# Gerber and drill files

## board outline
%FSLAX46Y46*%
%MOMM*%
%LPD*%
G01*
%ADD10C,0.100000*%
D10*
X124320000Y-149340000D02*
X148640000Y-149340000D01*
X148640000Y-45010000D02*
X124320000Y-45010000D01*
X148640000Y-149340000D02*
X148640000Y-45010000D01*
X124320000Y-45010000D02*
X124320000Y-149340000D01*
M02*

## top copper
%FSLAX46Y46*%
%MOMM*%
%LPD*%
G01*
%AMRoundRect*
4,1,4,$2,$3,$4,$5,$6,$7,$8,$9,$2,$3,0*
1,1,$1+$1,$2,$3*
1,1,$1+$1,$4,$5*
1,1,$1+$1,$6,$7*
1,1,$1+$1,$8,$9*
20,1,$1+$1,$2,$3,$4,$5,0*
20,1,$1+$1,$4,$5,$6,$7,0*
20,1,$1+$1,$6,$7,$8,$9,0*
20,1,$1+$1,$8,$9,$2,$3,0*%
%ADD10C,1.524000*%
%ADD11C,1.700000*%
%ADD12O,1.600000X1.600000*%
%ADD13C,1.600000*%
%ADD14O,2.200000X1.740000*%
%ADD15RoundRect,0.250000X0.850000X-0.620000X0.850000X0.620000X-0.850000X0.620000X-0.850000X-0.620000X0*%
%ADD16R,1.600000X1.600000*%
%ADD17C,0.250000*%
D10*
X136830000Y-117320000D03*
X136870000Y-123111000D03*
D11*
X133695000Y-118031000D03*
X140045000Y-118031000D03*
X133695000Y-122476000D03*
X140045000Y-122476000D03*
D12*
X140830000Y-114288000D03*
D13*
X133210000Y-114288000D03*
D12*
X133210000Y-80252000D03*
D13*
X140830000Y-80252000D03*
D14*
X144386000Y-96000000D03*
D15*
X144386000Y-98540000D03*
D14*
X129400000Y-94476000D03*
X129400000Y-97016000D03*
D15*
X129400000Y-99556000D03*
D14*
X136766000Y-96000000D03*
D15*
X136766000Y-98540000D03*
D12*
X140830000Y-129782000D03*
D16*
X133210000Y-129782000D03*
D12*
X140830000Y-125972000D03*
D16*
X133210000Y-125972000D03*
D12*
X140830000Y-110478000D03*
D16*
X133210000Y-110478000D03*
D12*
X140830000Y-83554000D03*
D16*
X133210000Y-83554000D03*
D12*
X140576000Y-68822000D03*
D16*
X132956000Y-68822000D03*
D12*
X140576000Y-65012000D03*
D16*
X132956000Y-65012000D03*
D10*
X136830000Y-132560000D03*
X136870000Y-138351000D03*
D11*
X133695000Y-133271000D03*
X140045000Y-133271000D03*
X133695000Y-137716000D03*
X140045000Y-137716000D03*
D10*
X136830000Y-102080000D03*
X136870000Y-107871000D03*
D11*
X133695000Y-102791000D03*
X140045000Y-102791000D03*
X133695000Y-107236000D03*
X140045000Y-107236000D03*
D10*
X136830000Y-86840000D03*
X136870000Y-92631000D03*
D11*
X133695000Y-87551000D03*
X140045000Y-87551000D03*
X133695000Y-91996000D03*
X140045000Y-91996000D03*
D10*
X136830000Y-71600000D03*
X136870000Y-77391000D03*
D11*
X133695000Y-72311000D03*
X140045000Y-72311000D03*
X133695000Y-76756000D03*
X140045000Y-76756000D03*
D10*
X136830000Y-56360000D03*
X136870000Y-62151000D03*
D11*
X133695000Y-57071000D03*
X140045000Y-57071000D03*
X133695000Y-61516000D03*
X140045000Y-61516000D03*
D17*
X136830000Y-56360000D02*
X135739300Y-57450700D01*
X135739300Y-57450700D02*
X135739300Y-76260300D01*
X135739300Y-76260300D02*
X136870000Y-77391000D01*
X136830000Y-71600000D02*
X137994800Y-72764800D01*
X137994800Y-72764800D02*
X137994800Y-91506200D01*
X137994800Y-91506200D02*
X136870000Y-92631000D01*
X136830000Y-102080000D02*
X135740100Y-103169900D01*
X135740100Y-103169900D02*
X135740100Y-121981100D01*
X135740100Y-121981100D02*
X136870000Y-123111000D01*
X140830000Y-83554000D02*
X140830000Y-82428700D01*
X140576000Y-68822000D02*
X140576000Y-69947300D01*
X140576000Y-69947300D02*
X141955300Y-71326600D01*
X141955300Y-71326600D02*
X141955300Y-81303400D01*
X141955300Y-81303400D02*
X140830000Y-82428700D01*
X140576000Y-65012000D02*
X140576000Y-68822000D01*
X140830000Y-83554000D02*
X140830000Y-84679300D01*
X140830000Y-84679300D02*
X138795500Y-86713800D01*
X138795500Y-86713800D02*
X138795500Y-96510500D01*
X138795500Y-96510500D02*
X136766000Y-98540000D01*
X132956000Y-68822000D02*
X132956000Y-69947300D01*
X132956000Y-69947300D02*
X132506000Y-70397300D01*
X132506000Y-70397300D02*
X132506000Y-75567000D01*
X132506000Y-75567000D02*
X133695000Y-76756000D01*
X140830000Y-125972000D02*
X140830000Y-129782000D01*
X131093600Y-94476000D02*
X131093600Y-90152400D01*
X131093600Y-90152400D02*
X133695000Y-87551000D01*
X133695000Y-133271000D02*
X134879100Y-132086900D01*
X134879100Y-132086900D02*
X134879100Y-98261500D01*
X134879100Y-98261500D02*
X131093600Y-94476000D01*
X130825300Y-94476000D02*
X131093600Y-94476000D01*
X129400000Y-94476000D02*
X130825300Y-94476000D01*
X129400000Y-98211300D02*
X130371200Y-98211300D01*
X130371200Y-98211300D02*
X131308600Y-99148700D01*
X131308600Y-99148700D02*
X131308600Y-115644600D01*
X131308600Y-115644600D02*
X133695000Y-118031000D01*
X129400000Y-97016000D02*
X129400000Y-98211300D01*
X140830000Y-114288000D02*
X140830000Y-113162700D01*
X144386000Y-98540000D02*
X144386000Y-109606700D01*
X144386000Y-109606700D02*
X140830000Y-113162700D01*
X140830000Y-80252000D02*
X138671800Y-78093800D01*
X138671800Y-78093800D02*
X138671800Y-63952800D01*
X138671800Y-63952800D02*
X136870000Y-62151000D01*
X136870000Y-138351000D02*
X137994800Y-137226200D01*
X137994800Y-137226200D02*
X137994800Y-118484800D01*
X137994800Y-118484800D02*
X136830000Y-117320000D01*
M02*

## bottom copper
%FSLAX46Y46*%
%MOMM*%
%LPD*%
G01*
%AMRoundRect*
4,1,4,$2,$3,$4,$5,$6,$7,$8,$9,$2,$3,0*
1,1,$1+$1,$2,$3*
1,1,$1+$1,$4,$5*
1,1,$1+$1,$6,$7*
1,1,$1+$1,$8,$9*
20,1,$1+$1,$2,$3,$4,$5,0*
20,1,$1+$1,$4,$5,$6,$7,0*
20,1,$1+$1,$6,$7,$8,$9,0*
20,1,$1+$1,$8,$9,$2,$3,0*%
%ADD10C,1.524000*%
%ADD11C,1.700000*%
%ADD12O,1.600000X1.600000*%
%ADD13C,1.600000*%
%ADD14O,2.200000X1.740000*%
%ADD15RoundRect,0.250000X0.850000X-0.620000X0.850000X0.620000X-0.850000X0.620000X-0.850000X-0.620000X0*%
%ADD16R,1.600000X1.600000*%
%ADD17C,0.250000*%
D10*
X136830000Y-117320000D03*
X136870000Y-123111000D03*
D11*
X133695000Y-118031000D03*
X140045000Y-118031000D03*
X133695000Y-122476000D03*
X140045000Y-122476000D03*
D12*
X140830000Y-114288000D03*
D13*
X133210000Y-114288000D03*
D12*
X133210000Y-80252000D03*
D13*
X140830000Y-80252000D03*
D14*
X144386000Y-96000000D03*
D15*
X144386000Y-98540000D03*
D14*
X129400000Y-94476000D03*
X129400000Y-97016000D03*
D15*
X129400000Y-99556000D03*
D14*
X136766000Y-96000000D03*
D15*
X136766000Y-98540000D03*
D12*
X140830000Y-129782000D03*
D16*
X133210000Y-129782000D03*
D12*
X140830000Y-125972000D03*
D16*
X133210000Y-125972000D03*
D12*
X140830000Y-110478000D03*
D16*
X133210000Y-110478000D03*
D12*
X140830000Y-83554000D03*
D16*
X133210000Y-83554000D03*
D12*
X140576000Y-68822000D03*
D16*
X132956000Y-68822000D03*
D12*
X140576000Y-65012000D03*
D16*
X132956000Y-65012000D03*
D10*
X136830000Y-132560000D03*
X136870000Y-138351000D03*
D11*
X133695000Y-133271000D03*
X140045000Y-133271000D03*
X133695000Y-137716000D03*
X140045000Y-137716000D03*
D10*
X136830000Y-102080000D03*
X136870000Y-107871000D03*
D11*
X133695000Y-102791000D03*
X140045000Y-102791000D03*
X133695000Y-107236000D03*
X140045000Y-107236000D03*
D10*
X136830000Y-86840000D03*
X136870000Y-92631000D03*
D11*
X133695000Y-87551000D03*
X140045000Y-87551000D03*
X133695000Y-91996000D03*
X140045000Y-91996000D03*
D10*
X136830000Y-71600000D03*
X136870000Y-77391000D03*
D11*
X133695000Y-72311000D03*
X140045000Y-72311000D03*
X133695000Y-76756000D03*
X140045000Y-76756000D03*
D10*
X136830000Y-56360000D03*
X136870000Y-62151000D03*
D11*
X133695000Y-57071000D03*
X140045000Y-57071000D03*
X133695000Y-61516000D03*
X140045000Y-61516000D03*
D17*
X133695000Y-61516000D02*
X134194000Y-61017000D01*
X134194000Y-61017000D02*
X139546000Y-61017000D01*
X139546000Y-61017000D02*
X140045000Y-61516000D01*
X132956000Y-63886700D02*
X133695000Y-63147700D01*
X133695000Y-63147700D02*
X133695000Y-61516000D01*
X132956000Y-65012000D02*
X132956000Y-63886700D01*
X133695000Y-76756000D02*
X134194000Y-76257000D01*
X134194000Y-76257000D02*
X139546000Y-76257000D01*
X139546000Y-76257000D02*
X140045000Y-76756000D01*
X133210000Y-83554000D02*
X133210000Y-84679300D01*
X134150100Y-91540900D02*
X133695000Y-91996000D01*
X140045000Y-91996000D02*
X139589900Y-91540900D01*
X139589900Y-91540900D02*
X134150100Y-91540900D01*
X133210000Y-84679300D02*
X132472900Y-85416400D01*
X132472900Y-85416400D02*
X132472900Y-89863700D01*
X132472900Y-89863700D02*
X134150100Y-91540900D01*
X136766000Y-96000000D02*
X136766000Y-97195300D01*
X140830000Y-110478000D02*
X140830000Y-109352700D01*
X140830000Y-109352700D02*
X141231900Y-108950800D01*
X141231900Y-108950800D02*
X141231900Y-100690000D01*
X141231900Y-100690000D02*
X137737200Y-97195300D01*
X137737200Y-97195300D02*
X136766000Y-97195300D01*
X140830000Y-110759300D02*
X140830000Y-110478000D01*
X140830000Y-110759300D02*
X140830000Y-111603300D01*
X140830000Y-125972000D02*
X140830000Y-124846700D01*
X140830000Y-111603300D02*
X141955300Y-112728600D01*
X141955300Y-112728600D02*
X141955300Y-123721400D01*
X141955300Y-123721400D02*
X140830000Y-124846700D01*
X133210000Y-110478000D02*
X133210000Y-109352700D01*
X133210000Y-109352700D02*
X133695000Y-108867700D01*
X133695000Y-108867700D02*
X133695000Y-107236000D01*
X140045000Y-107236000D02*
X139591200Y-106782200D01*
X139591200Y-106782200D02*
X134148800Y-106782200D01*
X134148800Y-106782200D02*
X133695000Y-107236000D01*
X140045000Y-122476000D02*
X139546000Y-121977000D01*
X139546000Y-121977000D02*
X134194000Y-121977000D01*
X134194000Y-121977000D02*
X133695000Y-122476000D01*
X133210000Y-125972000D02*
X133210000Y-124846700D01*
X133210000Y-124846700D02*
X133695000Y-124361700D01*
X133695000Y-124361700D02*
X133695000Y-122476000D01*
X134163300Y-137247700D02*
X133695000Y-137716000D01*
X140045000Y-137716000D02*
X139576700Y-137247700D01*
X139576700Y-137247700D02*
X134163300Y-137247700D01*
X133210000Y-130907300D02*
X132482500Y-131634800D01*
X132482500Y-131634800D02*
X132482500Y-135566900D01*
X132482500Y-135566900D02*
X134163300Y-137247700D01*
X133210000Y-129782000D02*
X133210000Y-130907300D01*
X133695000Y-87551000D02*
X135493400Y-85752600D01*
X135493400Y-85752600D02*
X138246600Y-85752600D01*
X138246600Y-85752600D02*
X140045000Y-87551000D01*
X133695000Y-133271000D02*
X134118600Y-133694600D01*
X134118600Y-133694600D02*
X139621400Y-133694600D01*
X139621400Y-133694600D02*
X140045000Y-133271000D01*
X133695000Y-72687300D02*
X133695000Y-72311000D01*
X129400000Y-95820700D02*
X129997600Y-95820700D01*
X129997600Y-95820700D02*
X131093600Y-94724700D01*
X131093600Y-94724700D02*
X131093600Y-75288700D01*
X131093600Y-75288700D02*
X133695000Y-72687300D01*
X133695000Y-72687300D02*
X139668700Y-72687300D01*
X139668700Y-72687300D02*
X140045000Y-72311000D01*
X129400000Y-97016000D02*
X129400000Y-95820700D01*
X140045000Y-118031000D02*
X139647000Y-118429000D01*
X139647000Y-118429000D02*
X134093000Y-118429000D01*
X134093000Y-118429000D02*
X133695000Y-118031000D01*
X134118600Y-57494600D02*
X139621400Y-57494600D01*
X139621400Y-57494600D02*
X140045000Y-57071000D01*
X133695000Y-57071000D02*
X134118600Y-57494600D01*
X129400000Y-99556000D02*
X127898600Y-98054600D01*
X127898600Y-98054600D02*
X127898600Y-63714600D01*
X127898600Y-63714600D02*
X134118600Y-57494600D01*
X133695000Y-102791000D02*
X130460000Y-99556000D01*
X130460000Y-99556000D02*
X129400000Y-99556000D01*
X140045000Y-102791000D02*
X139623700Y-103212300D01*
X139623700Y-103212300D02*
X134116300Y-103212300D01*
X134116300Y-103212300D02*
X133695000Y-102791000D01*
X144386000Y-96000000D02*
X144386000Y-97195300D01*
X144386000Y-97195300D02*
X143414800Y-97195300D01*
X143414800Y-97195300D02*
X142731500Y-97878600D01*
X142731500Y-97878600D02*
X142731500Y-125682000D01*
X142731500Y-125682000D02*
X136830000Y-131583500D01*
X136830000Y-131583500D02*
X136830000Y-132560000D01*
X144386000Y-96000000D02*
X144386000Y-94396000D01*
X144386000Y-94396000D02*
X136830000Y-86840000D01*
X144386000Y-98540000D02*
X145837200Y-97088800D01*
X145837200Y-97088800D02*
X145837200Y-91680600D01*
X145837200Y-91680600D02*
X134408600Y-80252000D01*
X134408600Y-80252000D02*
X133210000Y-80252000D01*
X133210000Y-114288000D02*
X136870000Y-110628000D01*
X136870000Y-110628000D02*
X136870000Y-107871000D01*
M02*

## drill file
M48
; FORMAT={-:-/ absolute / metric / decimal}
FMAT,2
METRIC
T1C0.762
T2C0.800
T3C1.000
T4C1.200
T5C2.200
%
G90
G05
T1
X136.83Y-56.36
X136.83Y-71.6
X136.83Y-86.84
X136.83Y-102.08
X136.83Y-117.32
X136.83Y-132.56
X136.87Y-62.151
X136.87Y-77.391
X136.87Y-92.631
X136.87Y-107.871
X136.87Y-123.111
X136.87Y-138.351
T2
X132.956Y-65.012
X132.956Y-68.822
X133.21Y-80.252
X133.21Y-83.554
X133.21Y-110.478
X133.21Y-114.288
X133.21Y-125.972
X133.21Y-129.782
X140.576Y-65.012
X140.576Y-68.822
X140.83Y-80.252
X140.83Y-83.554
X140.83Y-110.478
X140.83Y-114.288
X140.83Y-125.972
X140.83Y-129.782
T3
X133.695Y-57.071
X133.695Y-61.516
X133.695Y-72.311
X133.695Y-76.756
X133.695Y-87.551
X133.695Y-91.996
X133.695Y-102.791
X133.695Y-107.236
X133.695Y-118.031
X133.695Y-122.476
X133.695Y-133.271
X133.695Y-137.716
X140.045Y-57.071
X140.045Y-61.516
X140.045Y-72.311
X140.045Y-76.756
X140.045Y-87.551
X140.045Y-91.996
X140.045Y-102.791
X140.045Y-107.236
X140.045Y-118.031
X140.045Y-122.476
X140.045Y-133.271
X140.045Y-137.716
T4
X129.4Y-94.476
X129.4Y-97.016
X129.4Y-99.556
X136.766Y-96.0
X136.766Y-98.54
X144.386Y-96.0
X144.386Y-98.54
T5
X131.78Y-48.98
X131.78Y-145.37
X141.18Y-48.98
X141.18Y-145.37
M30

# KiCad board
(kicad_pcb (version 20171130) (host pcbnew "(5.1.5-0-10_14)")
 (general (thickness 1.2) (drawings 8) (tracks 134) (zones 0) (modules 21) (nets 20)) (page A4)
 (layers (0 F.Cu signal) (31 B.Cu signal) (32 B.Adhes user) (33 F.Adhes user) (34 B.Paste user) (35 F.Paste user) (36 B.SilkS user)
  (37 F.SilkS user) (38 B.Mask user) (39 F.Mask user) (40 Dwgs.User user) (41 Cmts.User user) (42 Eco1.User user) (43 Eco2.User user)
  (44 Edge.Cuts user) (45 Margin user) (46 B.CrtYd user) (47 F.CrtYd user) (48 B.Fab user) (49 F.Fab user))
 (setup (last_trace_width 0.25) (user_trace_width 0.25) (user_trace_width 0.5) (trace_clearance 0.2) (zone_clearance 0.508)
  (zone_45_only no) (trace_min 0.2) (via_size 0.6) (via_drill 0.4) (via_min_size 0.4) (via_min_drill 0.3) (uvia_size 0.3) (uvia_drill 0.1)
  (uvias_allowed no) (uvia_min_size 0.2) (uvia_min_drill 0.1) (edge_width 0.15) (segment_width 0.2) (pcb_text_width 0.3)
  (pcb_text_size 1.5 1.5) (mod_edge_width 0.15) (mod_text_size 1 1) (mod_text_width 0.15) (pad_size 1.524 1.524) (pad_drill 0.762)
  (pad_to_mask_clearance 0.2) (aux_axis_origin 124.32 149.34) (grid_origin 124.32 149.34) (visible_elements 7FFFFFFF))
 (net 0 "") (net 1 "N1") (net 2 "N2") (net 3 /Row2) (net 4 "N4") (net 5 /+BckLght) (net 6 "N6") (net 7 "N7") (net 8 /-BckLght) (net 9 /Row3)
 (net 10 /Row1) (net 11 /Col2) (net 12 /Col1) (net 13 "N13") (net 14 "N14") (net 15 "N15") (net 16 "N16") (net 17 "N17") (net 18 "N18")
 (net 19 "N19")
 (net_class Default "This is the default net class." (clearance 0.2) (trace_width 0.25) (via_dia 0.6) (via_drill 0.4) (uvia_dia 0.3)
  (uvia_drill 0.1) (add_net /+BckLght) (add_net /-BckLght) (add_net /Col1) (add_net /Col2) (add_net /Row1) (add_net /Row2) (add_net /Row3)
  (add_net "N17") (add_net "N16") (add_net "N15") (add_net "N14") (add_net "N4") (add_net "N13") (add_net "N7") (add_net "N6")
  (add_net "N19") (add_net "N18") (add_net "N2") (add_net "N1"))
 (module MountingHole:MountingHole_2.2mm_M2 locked (layer F.Cu) (at 141.18 48.98)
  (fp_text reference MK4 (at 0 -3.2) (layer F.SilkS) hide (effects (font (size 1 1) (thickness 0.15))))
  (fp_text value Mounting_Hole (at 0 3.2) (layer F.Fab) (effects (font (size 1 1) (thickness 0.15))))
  (pad 1 np_thru_hole circle (at 0 0) (size 2.2 2.2) (drill 2.2) (layers *.Cu *.Mask)))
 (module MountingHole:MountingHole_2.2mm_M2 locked (layer F.Cu) (at 131.78 48.98)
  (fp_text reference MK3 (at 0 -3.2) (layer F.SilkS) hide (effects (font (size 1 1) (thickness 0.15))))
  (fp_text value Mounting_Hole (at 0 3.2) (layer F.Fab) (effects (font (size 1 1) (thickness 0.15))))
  (pad 1 np_thru_hole circle (at 0 0) (size 2.2 2.2) (drill 2.2) (layers *.Cu *.Mask)))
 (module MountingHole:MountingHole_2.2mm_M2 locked (layer F.Cu) (at 141.18 145.37)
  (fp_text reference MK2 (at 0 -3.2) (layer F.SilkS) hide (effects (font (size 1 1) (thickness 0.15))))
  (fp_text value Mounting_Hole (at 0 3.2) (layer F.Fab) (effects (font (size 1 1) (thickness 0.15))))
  (pad 1 np_thru_hole circle (at 0 0) (size 2.2 2.2) (drill 2.2) (layers *.Cu *.Mask)))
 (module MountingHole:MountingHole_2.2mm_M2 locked (layer F.Cu) (at 131.78 145.37)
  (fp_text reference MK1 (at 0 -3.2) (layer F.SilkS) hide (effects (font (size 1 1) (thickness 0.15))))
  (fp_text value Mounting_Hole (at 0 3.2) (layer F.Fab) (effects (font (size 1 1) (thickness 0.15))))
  (pad 1 np_thru_hole circle (at 0 0) (size 2.2 2.2) (drill 2.2) (layers *.Cu *.Mask)))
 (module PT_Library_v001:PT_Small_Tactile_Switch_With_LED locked (layer F.Cu) (at 136.87 120.19 180)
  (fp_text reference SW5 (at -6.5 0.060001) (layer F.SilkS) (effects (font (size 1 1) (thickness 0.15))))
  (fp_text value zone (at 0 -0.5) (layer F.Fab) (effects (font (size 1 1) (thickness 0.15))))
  (pad 6 thru_hole circle (at 0.04 2.87 180) (size 1.524 1.524) (drill 0.762) (layers *.Cu *.Mask) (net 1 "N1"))
  (pad 5 thru_hole circle (at 0 -2.921 180) (size 1.524 1.524) (drill 0.762) (layers *.Cu *.Mask) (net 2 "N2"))
  (pad 4 thru_hole circle (at 3.175 2.159 180) (size 1.7 1.7) (drill 1) (layers *.Cu *.Mask) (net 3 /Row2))
  (pad 3 thru_hole circle (at -3.175 2.159 180) (size 1.7 1.7) (drill 1) (layers *.Cu *.Mask) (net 3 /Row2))
  (pad 2 thru_hole circle (at 3.175 -2.286 180) (size 1.7 1.7) (drill 1) (layers *.Cu *.Mask) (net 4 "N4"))
  (pad 1 thru_hole circle (at -3.175 -2.286 180) (size 1.7 1.7) (drill 1) (layers *.Cu *.Mask) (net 4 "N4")))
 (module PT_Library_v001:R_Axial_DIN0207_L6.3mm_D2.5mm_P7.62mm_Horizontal (layer F.Cu) (at 133.21 114.288)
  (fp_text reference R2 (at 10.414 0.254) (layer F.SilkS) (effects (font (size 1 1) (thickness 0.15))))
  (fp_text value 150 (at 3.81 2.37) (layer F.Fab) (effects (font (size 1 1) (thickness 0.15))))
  (pad 2 thru_hole oval (at 7.62 0) (size 1.6 1.6) (drill 0.8) (layers *.Cu *.Mask) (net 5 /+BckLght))
  (pad 1 thru_hole circle (at 0 0) (size 1.6 1.6) (drill 0.8) (layers *.Cu *.Mask) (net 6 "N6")))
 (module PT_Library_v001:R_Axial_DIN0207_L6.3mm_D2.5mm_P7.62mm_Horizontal (layer F.Cu) (at 140.83 80.252 180)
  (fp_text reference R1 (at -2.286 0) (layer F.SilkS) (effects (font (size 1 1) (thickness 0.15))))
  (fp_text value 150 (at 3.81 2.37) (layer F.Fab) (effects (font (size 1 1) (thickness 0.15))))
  (pad 2 thru_hole oval (at 7.62 0 180) (size 1.6 1.6) (drill 0.8) (layers *.Cu *.Mask) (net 5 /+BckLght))
  (pad 1 thru_hole circle (at 0 0 180) (size 1.6 1.6) (drill 0.8) (layers *.Cu *.Mask) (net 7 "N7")))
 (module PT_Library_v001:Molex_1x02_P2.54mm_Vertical (layer F.Cu) (at 144.386 98.54 90)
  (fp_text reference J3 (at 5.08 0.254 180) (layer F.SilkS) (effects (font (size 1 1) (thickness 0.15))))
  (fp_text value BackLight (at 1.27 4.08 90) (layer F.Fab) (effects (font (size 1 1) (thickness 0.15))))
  (pad 2 thru_hole oval (at 2.54 0 90) (size 1.74 2.2) (drill 1.2) (layers *.Cu *.Mask) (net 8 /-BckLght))
  (pad 1 thru_hole roundrect (at 0 0 90) (size 1.74 2.2) (drill 1.2) (layers *.Cu *.Mask) (roundrect_rratio 0.143678) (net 5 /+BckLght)))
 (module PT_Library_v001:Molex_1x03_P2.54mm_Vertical (layer F.Cu) (at 129.4 99.556 90)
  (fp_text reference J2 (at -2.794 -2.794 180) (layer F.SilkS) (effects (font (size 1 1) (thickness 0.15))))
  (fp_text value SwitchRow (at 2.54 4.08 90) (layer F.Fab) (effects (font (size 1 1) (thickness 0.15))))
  (pad 3 thru_hole oval (at 5.08 0 90) (size 1.74 2.2) (drill 1.2) (layers *.Cu *.Mask) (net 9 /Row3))
  (pad 2 thru_hole oval (at 2.54 0 90) (size 1.74 2.2) (drill 1.2) (layers *.Cu *.Mask) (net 3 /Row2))
  (pad 1 thru_hole roundrect (at 0 0 90) (size 1.74 2.2) (drill 1.2) (layers *.Cu *.Mask) (roundrect_rratio 0.143678) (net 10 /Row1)))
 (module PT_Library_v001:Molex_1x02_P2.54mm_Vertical (layer F.Cu) (at 136.766 98.54 90)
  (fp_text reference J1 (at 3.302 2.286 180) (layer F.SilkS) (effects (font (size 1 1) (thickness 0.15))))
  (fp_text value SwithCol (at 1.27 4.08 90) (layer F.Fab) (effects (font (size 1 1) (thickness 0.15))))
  (pad 2 thru_hole oval (at 2.54 0 90) (size 1.74 2.2) (drill 1.2) (layers *.Cu *.Mask) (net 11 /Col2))
  (pad 1 thru_hole roundrect (at 0 0 90) (size 1.74 2.2) (drill 1.2) (layers *.Cu *.Mask) (roundrect_rratio 0.143678) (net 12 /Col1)))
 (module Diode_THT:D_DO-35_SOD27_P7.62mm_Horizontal (layer F.Cu) (at 133.21 129.782)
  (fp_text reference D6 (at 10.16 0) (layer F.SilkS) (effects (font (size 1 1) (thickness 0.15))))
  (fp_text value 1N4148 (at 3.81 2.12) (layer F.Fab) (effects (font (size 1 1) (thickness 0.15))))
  (pad 2 thru_hole oval (at 7.62 0) (size 1.6 1.6) (drill 0.8) (layers *.Cu *.Mask) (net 11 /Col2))
  (pad 1 thru_hole rect (at 0 0) (size 1.6 1.6) (drill 0.8) (layers *.Cu *.Mask) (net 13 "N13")))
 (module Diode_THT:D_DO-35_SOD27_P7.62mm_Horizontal (layer F.Cu) (at 133.21 125.972)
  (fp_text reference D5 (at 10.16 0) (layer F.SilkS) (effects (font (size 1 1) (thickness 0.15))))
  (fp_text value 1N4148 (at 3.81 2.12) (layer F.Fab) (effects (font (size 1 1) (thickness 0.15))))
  (pad 2 thru_hole oval (at 7.62 0) (size 1.6 1.6) (drill 0.8) (layers *.Cu *.Mask) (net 11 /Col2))
  (pad 1 thru_hole rect (at 0 0) (size 1.6 1.6) (drill 0.8) (layers *.Cu *.Mask) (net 4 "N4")))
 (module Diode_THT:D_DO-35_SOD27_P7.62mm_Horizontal (layer F.Cu) (at 133.21 110.478)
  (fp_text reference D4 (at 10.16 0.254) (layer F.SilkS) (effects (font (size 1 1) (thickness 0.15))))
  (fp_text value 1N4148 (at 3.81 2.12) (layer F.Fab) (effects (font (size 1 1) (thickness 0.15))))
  (pad 2 thru_hole oval (at 7.62 0) (size 1.6 1.6) (drill 0.8) (layers *.Cu *.Mask) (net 11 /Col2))
  (pad 1 thru_hole rect (at 0 0) (size 1.6 1.6) (drill 0.8) (layers *.Cu *.Mask) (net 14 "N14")))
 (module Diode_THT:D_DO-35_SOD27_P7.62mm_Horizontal (layer F.Cu) (at 133.21 83.554)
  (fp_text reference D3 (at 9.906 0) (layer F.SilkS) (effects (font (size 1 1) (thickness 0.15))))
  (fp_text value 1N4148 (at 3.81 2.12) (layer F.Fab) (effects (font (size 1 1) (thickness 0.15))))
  (pad 2 thru_hole oval (at 7.62 0) (size 1.6 1.6) (drill 0.8) (layers *.Cu *.Mask) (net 12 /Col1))
  (pad 1 thru_hole rect (at 0 0) (size 1.6 1.6) (drill 0.8) (layers *.Cu *.Mask) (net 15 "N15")))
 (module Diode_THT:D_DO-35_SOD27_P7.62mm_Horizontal (layer F.Cu) (at 132.956 68.822)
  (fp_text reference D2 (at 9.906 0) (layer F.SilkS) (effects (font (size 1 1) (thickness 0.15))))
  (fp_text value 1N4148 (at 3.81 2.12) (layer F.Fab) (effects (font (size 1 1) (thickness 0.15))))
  (pad 2 thru_hole oval (at 7.62 0) (size 1.6 1.6) (drill 0.8) (layers *.Cu *.Mask) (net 12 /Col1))
  (pad 1 thru_hole rect (at 0 0) (size 1.6 1.6) (drill 0.8) (layers *.Cu *.Mask) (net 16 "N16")))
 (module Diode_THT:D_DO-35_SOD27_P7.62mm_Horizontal (layer F.Cu) (at 132.956 65.012)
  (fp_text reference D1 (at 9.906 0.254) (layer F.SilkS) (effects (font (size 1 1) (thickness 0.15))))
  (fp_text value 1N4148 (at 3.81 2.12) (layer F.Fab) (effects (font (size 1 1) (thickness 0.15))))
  (pad 2 thru_hole oval (at 7.62 0) (size 1.6 1.6) (drill 0.8) (layers *.Cu *.Mask) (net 12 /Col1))
  (pad 1 thru_hole rect (at 0 0) (size 1.6 1.6) (drill 0.8) (layers *.Cu *.Mask) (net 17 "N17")))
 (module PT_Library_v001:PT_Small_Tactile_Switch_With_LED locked (layer F.Cu) (at 136.87 135.43 180)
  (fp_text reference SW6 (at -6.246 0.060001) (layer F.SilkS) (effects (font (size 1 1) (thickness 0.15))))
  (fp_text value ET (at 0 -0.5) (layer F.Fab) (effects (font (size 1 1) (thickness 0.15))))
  (pad 6 thru_hole circle (at 0.04 2.87 180) (size 1.524 1.524) (drill 0.762) (layers *.Cu *.Mask) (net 8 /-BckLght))
  (pad 5 thru_hole circle (at 0 -2.921 180) (size 1.524 1.524) (drill 0.762) (layers *.Cu *.Mask) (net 1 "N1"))
  (pad 4 thru_hole circle (at 3.175 2.159 180) (size 1.7 1.7) (drill 1) (layers *.Cu *.Mask) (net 9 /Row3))
  (pad 3 thru_hole circle (at -3.175 2.159 180) (size 1.7 1.7) (drill 1) (layers *.Cu *.Mask) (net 9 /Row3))
  (pad 2 thru_hole circle (at 3.175 -2.286 180) (size 1.7 1.7) (drill 1) (layers *.Cu *.Mask) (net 13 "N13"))
  (pad 1 thru_hole circle (at -3.175 -2.286 180) (size 1.7 1.7) (drill 1) (layers *.Cu *.Mask) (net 13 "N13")))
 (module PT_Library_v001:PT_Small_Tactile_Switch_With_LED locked (layer F.Cu) (at 136.87 104.95 180)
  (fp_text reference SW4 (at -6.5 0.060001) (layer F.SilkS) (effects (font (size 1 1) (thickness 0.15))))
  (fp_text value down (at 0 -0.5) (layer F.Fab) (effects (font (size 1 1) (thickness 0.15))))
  (pad 6 thru_hole circle (at 0.04 2.87 180) (size 1.524 1.524) (drill 0.762) (layers *.Cu *.Mask) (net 2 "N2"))
  (pad 5 thru_hole circle (at 0 -2.921 180) (size 1.524 1.524) (drill 0.762) (layers *.Cu *.Mask) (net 6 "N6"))
  (pad 4 thru_hole circle (at 3.175 2.159 180) (size 1.7 1.7) (drill 1) (layers *.Cu *.Mask) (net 10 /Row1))
  (pad 3 thru_hole circle (at -3.175 2.159 180) (size 1.7 1.7) (drill 1) (layers *.Cu *.Mask) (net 10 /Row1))
  (pad 2 thru_hole circle (at 3.175 -2.286 180) (size 1.7 1.7) (drill 1) (layers *.Cu *.Mask) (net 14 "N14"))
  (pad 1 thru_hole circle (at -3.175 -2.286 180) (size 1.7 1.7) (drill 1) (layers *.Cu *.Mask) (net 14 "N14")))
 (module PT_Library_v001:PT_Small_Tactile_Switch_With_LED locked (layer F.Cu) (at 136.87 89.71 180)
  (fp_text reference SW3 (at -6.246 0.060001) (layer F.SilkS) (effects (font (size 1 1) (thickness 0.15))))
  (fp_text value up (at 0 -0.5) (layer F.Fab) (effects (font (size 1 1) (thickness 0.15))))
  (pad 6 thru_hole circle (at 0.04 2.87 180) (size 1.524 1.524) (drill 0.762) (layers *.Cu *.Mask) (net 8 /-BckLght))
  (pad 5 thru_hole circle (at 0 -2.921 180) (size 1.524 1.524) (drill 0.762) (layers *.Cu *.Mask) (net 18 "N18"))
  (pad 4 thru_hole circle (at 3.175 2.159 180) (size 1.7 1.7) (drill 1) (layers *.Cu *.Mask) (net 9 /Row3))
  (pad 3 thru_hole circle (at -3.175 2.159 180) (size 1.7 1.7) (drill 1) (layers *.Cu *.Mask) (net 9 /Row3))
  (pad 2 thru_hole circle (at 3.175 -2.286 180) (size 1.7 1.7) (drill 1) (layers *.Cu *.Mask) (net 15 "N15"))
  (pad 1 thru_hole circle (at -3.175 -2.286 180) (size 1.7 1.7) (drill 1) (layers *.Cu *.Mask) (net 15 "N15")))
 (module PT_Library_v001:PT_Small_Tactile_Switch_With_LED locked (layer F.Cu) (at 136.87 74.47 180)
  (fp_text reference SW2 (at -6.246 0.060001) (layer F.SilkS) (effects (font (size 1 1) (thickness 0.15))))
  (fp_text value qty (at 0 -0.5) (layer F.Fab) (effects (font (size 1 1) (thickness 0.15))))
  (pad 6 thru_hole circle (at 0.04 2.87 180) (size 1.524 1.524) (drill 0.762) (layers *.Cu *.Mask) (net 18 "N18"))
  (pad 5 thru_hole circle (at 0 -2.921 180) (size 1.524 1.524) (drill 0.762) (layers *.Cu *.Mask) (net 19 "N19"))
  (pad 4 thru_hole circle (at 3.175 2.159 180) (size 1.7 1.7) (drill 1) (layers *.Cu *.Mask) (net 3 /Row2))
  (pad 3 thru_hole circle (at -3.175 2.159 180) (size 1.7 1.7) (drill 1) (layers *.Cu *.Mask) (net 3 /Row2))
  (pad 2 thru_hole circle (at 3.175 -2.286 180) (size 1.7 1.7) (drill 1) (layers *.Cu *.Mask) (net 16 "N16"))
  (pad 1 thru_hole circle (at -3.175 -2.286 180) (size 1.7 1.7) (drill 1) (layers *.Cu *.Mask) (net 16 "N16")))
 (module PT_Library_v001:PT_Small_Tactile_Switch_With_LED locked (layer F.Cu) (at 136.87 59.23 180)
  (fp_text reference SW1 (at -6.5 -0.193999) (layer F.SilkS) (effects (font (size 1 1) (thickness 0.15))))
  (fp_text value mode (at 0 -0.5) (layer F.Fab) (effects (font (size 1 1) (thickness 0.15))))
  (pad 6 thru_hole circle (at 0.04 2.87 180) (size 1.524 1.524) (drill 0.762) (layers *.Cu *.Mask) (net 19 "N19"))
  (pad 5 thru_hole circle (at 0 -2.921 180) (size 1.524 1.524) (drill 0.762) (layers *.Cu *.Mask) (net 7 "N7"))
  (pad 4 thru_hole circle (at 3.175 2.159 180) (size 1.7 1.7) (drill 1) (layers *.Cu *.Mask) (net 10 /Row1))
  (pad 3 thru_hole circle (at -3.175 2.159 180) (size 1.7 1.7) (drill 1) (layers *.Cu *.Mask) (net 10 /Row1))
  (pad 2 thru_hole circle (at 3.175 -2.286 180) (size 1.7 1.7) (drill 1) (layers *.Cu *.Mask) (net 17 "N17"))
  (pad 1 thru_hole circle (at -3.175 -2.286 180) (size 1.7 1.7) (drill 1) (layers *.Cu *.Mask) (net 17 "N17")))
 (gr_line (start 124.32 149.34) (end 148.64 149.34) (layer Edge.Cuts) (width 0.1))
 (gr_line (start 148.64 45.01) (end 124.32 45.01) (layer Edge.Cuts) (width 0.1))
 (gr_line (start 148.64 149.34) (end 148.64 45.01) (layer Edge.Cuts) (width 0.1))
 (gr_line (start 124.32 45.01) (end 124.32 149.34) (layer Edge.Cuts) (width 0.1))
 (segment (start 136.83 56.36) (end 135.7393 57.4507) (width 0.25) (layer F.Cu) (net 19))
 (segment (start 135.7393 57.4507) (end 135.7393 76.2603) (width 0.25) (layer F.Cu) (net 19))
 (segment (start 135.7393 76.2603) (end 136.87 77.391) (width 0.25) (layer F.Cu) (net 19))
 (segment (start 136.83 71.6) (end 137.9948 72.7648) (width 0.25) (layer F.Cu) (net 18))
 (segment (start 137.9948 72.7648) (end 137.9948 91.5062) (width 0.25) (layer F.Cu) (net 18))
 (segment (start 137.9948 91.5062) (end 136.87 92.631) (width 0.25) (layer F.Cu) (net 18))
 (segment (start 136.83 102.08) (end 135.7401 103.1699) (width 0.25) (layer F.Cu) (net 2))
 (segment (start 135.7401 103.1699) (end 135.7401 121.9811) (width 0.25) (layer F.Cu) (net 2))
 (segment (start 135.7401 121.9811) (end 136.87 123.111) (width 0.25) (layer F.Cu) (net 2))
 (segment (start 140.83 83.554) (end 140.83 82.4287) (width 0.25) (layer F.Cu) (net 12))
 (segment (start 140.576 68.822) (end 140.576 69.9473) (width 0.25) (layer F.Cu) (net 12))
 (segment (start 140.576 69.9473) (end 141.9553 71.3266) (width 0.25) (layer F.Cu) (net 12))
 (segment (start 141.9553 71.3266) (end 141.9553 81.3034) (width 0.25) (layer F.Cu) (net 12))
 (segment (start 141.9553 81.3034) (end 140.83 82.4287) (width 0.25) (layer F.Cu) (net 12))
 (segment (start 140.576 65.012) (end 140.576 68.822) (width 0.25) (layer F.Cu) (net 12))
 (segment (start 140.83 83.554) (end 140.83 84.6793) (width 0.25) (layer F.Cu) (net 12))
 (segment (start 140.83 84.6793) (end 138.7955 86.7138) (width 0.25) (layer F.Cu) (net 12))
 (segment (start 138.7955 86.7138) (end 138.7955 96.5105) (width 0.25) (layer F.Cu) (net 12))
 (segment (start 138.7955 96.5105) (end 136.766 98.54) (width 0.25) (layer F.Cu) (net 12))
 (segment (start 133.695 61.516) (end 134.194 61.017) (width 0.25) (layer B.Cu) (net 17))
 (segment (start 134.194 61.017) (end 139.546 61.017) (width 0.25) (layer B.Cu) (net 17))
 (segment (start 139.546 61.017) (end 140.045 61.516) (width 0.25) (layer B.Cu) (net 17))
 (segment (start 132.956 63.8867) (end 133.695 63.1477) (width 0.25) (layer B.Cu) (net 17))
 (segment (start 133.695 63.1477) (end 133.695 61.516) (width 0.25) (layer B.Cu) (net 17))
 (segment (start 132.956 65.012) (end 132.956 63.8867) (width 0.25) (layer B.Cu) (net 17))
 (segment (start 132.956 68.822) (end 132.956 69.9473) (width 0.25) (layer F.Cu) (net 16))
 (segment (start 132.956 69.9473) (end 132.506 70.3973) (width 0.25) (layer F.Cu) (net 16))
 (segment (start 132.506 70.3973) (end 132.506 75.567) (width 0.25) (layer F.Cu) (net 16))
 (segment (start 132.506 75.567) (end 133.695 76.756) (width 0.25) (layer F.Cu) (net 16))
 (segment (start 133.695 76.756) (end 134.194 76.257) (width 0.25) (layer B.Cu) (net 16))
 (segment (start 134.194 76.257) (end 139.546 76.257) (width 0.25) (layer B.Cu) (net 16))
 (segment (start 139.546 76.257) (end 140.045 76.756) (width 0.25) (layer B.Cu) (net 16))
 (segment (start 133.21 83.554) (end 133.21 84.6793) (width 0.25) (layer B.Cu) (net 15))
 (segment (start 134.1501 91.5409) (end 133.695 91.996) (width 0.25) (layer B.Cu) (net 15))
 (segment (start 140.045 91.996) (end 139.5899 91.5409) (width 0.25) (layer B.Cu) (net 15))
 (segment (start 139.5899 91.5409) (end 134.1501 91.5409) (width 0.25) (layer B.Cu) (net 15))
 (segment (start 133.21 84.6793) (end 132.4729 85.4164) (width 0.25) (layer B.Cu) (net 15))
 (segment (start 132.4729 85.4164) (end 132.4729 89.8637) (width 0.25) (layer B.Cu) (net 15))
 (segment (start 132.4729 89.8637) (end 134.1501 91.5409) (width 0.25) (layer B.Cu) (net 15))
 (segment (start 136.766 96) (end 136.766 97.1953) (width 0.25) (layer B.Cu) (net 11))
 (segment (start 140.83 110.478) (end 140.83 109.3527) (width 0.25) (layer B.Cu) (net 11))
 (segment (start 140.83 109.3527) (end 141.2319 108.9508) (width 0.25) (layer B.Cu) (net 11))
 (segment (start 141.2319 108.9508) (end 141.2319 100.69) (width 0.25) (layer B.Cu) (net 11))
 (segment (start 141.2319 100.69) (end 137.7372 97.1953) (width 0.25) (layer B.Cu) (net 11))
 (segment (start 137.7372 97.1953) (end 136.766 97.1953) (width 0.25) (layer B.Cu) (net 11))
 (segment (start 140.83 110.7593) (end 140.83 110.478) (width 0.25) (layer B.Cu) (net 11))
 (segment (start 140.83 110.7593) (end 140.83 111.6033) (width 0.25) (layer B.Cu) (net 11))
 (segment (start 140.83 125.972) (end 140.83 129.782) (width 0.25) (layer F.Cu) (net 11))
 (segment (start 140.83 125.972) (end 140.83 124.8467) (width 0.25) (layer B.Cu) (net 11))
 (segment (start 140.83 111.6033) (end 141.9553 112.7286) (width 0.25) (layer B.Cu) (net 11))
 (segment (start 141.9553 112.7286) (end 141.9553 123.7214) (width 0.25) (layer B.Cu) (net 11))
 (segment (start 141.9553 123.7214) (end 140.83 124.8467) (width 0.25) (layer B.Cu) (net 11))
 (segment (start 133.21 110.478) (end 133.21 109.3527) (width 0.25) (layer B.Cu) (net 14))
 (segment (start 133.21 109.3527) (end 133.695 108.8677) (width 0.25) (layer B.Cu) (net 14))
 (segment (start 133.695 108.8677) (end 133.695 107.236) (width 0.25) (layer B.Cu) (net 14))
 (segment (start 140.045 107.236) (end 139.5912 106.7822) (width 0.25) (layer B.Cu) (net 14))
 (segment (start 139.5912 106.7822) (end 134.1488 106.7822) (width 0.25) (layer B.Cu) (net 14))
 (segment (start 134.1488 106.7822) (end 133.695 107.236) (width 0.25) (layer B.Cu) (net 14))
 (segment (start 140.045 122.476) (end 139.546 121.977) (width 0.25) (layer B.Cu) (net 4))
 (segment (start 139.546 121.977) (end 134.194 121.977) (width 0.25) (layer B.Cu) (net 4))
 (segment (start 134.194 121.977) (end 133.695 122.476) (width 0.25) (layer B.Cu) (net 4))
 (segment (start 133.21 125.972) (end 133.21 124.8467) (width 0.25) (layer B.Cu) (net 4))
 (segment (start 133.21 124.8467) (end 133.695 124.3617) (width 0.25) (layer B.Cu) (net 4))
 (segment (start 133.695 124.3617) (end 133.695 122.476) (width 0.25) (layer B.Cu) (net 4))
 (segment (start 134.1633 137.2477) (end 133.695 137.716) (width 0.25) (layer B.Cu) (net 13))
 (segment (start 140.045 137.716) (end 139.5767 137.2477) (width 0.25) (layer B.Cu) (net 13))
 (segment (start 139.5767 137.2477) (end 134.1633 137.2477) (width 0.25) (layer B.Cu) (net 13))
 (segment (start 133.21 130.9073) (end 132.4825 131.6348) (width 0.25) (layer B.Cu) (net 13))
 (segment (start 132.4825 131.6348) (end 132.4825 135.5669) (width 0.25) (layer B.Cu) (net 13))
 (segment (start 132.4825 135.5669) (end 134.1633 137.2477) (width 0.25) (layer B.Cu) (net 13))
 (segment (start 133.21 129.782) (end 133.21 130.9073) (width 0.25) (layer B.Cu) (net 13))
 (segment (start 131.0936 94.476) (end 131.0936 90.1524) (width 0.25) (layer F.Cu) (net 9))
 (segment (start 131.0936 90.1524) (end 133.695 87.551) (width 0.25) (layer F.Cu) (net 9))
 (segment (start 133.695 133.271) (end 134.8791 132.0869) (width 0.25) (layer F.Cu) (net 9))
 (segment (start 134.8791 132.0869) (end 134.8791 98.2615) (width 0.25) (layer F.Cu) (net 9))
 (segment (start 134.8791 98.2615) (end 131.0936 94.476) (width 0.25) (layer F.Cu) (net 9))
 (segment (start 130.8253 94.476) (end 131.0936 94.476) (width 0.25) (layer F.Cu) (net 9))
 (segment (start 129.4 94.476) (end 130.8253 94.476) (width 0.25) (layer F.Cu) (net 9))
 (segment (start 133.695 87.551) (end 135.4934 85.7526) (width 0.25) (layer B.Cu) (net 9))
 (segment (start 135.4934 85.7526) (end 138.2466 85.7526) (width 0.25) (layer B.Cu) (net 9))
 (segment (start 138.2466 85.7526) (end 140.045 87.551) (width 0.25) (layer B.Cu) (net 9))
 (segment (start 133.695 133.271) (end 134.1186 133.6946) (width 0.25) (layer B.Cu) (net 9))
 (segment (start 134.1186 133.6946) (end 139.6214 133.6946) (width 0.25) (layer B.Cu) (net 9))
 (segment (start 139.6214 133.6946) (end 140.045 133.271) (width 0.25) (layer B.Cu) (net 9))
 (segment (start 129.4 98.2113) (end 130.3712 98.2113) (width 0.25) (layer F.Cu) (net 3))
 (segment (start 130.3712 98.2113) (end 131.3086 99.1487) (width 0.25) (layer F.Cu) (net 3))
 (segment (start 131.3086 99.1487) (end 131.3086 115.6446) (width 0.25) (layer F.Cu) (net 3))
 (segment (start 131.3086 115.6446) (end 133.695 118.031) (width 0.25) (layer F.Cu) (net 3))
 (segment (start 133.695 72.6873) (end 133.695 72.311) (width 0.25) (layer B.Cu) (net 3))
 (segment (start 129.4 95.8207) (end 129.9976 95.8207) (width 0.25) (layer B.Cu) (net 3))
 (segment (start 129.9976 95.8207) (end 131.0936 94.7247) (width 0.25) (layer B.Cu) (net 3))
 (segment (start 131.0936 94.7247) (end 131.0936 75.2887) (width 0.25) (layer B.Cu) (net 3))
 (segment (start 131.0936 75.2887) (end 133.695 72.6873) (width 0.25) (layer B.Cu) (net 3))
 (segment (start 133.695 72.6873) (end 139.6687 72.6873) (width 0.25) (layer B.Cu) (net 3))
 (segment (start 139.6687 72.6873) (end 140.045 72.311) (width 0.25) (layer B.Cu) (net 3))
 (segment (start 129.4 97.016) (end 129.4 95.8207) (width 0.25) (layer B.Cu) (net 3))
 (segment (start 129.4 97.016) (end 129.4 98.2113) (width 0.25) (layer F.Cu) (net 3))
 (segment (start 140.045 118.031) (end 139.647 118.429) (width 0.25) (layer B.Cu) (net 3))
 (segment (start 139.647 118.429) (end 134.093 118.429) (width 0.25) (layer B.Cu) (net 3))
 (segment (start 134.093 118.429) (end 133.695 118.031) (width 0.25) (layer B.Cu) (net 3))
 (segment (start 134.1186 57.4946) (end 139.6214 57.4946) (width 0.25) (layer B.Cu) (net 10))
 (segment (start 139.6214 57.4946) (end 140.045 57.071) (width 0.25) (layer B.Cu) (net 10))
 (segment (start 133.695 57.071) (end 134.1186 57.4946) (width 0.25) (layer B.Cu) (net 10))
 (segment (start 129.4 99.556) (end 127.8986 98.0546) (width 0.25) (layer B.Cu) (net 10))
 (segment (start 127.8986 98.0546) (end 127.8986 63.7146) (width 0.25) (layer B.Cu) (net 10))
 (segment (start 127.8986 63.7146) (end 134.1186 57.4946) (width 0.25) (layer B.Cu) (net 10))
 (segment (start 133.695 102.791) (end 130.46 99.556) (width 0.25) (layer B.Cu) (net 10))
 (segment (start 130.46 99.556) (end 129.4 99.556) (width 0.25) (layer B.Cu) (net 10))
 (segment (start 140.045 102.791) (end 139.6237 103.2123) (width 0.25) (layer B.Cu) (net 10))
 (segment (start 139.6237 103.2123) (end 134.1163 103.2123) (width 0.25) (layer B.Cu) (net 10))
 (segment (start 134.1163 103.2123) (end 133.695 102.791) (width 0.25) (layer B.Cu) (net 10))
 (segment (start 144.386 96) (end 144.386 97.1953) (width 0.25) (layer B.Cu) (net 8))
 (segment (start 144.386 97.1953) (end 143.4148 97.1953) (width 0.25) (layer B.Cu) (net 8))
 (segment (start 143.4148 97.1953) (end 142.7315 97.8786) (width 0.25) (layer B.Cu) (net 8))
 (segment (start 142.7315 97.8786) (end 142.7315 125.682) (width 0.25) (layer B.Cu) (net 8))
 (segment (start 142.7315 125.682) (end 136.83 131.5835) (width 0.25) (layer B.Cu) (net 8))
 (segment (start 136.83 131.5835) (end 136.83 132.56) (width 0.25) (layer B.Cu) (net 8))
 (segment (start 144.386 96) (end 144.386 94.396) (width 0.25) (layer B.Cu) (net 8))
 (segment (start 144.386 94.396) (end 136.83 86.84) (width 0.25) (layer B.Cu) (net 8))
 (segment (start 144.386 98.54) (end 145.8372 97.0888) (width 0.25) (layer B.Cu) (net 5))
 (segment (start 145.8372 97.0888) (end 145.8372 91.6806) (width 0.25) (layer B.Cu) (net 5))
 (segment (start 145.8372 91.6806) (end 134.4086 80.252) (width 0.25) (layer B.Cu) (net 5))
 (segment (start 134.4086 80.252) (end 133.21 80.252) (width 0.25) (layer B.Cu) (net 5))
 (segment (start 140.83 114.288) (end 140.83 113.1627) (width 0.25) (layer F.Cu) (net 5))
 (segment (start 144.386 98.54) (end 144.386 109.6067) (width 0.25) (layer F.Cu) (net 5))
 (segment (start 144.386 109.6067) (end 140.83 113.1627) (width 0.25) (layer F.Cu) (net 5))
 (segment (start 140.83 80.252) (end 138.6718 78.0938) (width 0.25) (layer F.Cu) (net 7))
 (segment (start 138.6718 78.0938) (end 138.6718 63.9528) (width 0.25) (layer F.Cu) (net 7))
 (segment (start 138.6718 63.9528) (end 136.87 62.151) (width 0.25) (layer F.Cu) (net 7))
 (segment (start 133.21 114.288) (end 136.87 110.628) (width 0.25) (layer B.Cu) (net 6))
 (segment (start 136.87 110.628) (end 136.87 107.871) (width 0.25) (layer B.Cu) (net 6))
 (segment (start 136.87 138.351) (end 137.9948 137.2262) (width 0.25) (layer F.Cu) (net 1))
 (segment (start 137.9948 137.2262) (end 137.9948 118.4848) (width 0.25) (layer F.Cu) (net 1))
 (segment (start 137.9948 118.4848) (end 136.83 117.32) (width 0.25) (layer F.Cu) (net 1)))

